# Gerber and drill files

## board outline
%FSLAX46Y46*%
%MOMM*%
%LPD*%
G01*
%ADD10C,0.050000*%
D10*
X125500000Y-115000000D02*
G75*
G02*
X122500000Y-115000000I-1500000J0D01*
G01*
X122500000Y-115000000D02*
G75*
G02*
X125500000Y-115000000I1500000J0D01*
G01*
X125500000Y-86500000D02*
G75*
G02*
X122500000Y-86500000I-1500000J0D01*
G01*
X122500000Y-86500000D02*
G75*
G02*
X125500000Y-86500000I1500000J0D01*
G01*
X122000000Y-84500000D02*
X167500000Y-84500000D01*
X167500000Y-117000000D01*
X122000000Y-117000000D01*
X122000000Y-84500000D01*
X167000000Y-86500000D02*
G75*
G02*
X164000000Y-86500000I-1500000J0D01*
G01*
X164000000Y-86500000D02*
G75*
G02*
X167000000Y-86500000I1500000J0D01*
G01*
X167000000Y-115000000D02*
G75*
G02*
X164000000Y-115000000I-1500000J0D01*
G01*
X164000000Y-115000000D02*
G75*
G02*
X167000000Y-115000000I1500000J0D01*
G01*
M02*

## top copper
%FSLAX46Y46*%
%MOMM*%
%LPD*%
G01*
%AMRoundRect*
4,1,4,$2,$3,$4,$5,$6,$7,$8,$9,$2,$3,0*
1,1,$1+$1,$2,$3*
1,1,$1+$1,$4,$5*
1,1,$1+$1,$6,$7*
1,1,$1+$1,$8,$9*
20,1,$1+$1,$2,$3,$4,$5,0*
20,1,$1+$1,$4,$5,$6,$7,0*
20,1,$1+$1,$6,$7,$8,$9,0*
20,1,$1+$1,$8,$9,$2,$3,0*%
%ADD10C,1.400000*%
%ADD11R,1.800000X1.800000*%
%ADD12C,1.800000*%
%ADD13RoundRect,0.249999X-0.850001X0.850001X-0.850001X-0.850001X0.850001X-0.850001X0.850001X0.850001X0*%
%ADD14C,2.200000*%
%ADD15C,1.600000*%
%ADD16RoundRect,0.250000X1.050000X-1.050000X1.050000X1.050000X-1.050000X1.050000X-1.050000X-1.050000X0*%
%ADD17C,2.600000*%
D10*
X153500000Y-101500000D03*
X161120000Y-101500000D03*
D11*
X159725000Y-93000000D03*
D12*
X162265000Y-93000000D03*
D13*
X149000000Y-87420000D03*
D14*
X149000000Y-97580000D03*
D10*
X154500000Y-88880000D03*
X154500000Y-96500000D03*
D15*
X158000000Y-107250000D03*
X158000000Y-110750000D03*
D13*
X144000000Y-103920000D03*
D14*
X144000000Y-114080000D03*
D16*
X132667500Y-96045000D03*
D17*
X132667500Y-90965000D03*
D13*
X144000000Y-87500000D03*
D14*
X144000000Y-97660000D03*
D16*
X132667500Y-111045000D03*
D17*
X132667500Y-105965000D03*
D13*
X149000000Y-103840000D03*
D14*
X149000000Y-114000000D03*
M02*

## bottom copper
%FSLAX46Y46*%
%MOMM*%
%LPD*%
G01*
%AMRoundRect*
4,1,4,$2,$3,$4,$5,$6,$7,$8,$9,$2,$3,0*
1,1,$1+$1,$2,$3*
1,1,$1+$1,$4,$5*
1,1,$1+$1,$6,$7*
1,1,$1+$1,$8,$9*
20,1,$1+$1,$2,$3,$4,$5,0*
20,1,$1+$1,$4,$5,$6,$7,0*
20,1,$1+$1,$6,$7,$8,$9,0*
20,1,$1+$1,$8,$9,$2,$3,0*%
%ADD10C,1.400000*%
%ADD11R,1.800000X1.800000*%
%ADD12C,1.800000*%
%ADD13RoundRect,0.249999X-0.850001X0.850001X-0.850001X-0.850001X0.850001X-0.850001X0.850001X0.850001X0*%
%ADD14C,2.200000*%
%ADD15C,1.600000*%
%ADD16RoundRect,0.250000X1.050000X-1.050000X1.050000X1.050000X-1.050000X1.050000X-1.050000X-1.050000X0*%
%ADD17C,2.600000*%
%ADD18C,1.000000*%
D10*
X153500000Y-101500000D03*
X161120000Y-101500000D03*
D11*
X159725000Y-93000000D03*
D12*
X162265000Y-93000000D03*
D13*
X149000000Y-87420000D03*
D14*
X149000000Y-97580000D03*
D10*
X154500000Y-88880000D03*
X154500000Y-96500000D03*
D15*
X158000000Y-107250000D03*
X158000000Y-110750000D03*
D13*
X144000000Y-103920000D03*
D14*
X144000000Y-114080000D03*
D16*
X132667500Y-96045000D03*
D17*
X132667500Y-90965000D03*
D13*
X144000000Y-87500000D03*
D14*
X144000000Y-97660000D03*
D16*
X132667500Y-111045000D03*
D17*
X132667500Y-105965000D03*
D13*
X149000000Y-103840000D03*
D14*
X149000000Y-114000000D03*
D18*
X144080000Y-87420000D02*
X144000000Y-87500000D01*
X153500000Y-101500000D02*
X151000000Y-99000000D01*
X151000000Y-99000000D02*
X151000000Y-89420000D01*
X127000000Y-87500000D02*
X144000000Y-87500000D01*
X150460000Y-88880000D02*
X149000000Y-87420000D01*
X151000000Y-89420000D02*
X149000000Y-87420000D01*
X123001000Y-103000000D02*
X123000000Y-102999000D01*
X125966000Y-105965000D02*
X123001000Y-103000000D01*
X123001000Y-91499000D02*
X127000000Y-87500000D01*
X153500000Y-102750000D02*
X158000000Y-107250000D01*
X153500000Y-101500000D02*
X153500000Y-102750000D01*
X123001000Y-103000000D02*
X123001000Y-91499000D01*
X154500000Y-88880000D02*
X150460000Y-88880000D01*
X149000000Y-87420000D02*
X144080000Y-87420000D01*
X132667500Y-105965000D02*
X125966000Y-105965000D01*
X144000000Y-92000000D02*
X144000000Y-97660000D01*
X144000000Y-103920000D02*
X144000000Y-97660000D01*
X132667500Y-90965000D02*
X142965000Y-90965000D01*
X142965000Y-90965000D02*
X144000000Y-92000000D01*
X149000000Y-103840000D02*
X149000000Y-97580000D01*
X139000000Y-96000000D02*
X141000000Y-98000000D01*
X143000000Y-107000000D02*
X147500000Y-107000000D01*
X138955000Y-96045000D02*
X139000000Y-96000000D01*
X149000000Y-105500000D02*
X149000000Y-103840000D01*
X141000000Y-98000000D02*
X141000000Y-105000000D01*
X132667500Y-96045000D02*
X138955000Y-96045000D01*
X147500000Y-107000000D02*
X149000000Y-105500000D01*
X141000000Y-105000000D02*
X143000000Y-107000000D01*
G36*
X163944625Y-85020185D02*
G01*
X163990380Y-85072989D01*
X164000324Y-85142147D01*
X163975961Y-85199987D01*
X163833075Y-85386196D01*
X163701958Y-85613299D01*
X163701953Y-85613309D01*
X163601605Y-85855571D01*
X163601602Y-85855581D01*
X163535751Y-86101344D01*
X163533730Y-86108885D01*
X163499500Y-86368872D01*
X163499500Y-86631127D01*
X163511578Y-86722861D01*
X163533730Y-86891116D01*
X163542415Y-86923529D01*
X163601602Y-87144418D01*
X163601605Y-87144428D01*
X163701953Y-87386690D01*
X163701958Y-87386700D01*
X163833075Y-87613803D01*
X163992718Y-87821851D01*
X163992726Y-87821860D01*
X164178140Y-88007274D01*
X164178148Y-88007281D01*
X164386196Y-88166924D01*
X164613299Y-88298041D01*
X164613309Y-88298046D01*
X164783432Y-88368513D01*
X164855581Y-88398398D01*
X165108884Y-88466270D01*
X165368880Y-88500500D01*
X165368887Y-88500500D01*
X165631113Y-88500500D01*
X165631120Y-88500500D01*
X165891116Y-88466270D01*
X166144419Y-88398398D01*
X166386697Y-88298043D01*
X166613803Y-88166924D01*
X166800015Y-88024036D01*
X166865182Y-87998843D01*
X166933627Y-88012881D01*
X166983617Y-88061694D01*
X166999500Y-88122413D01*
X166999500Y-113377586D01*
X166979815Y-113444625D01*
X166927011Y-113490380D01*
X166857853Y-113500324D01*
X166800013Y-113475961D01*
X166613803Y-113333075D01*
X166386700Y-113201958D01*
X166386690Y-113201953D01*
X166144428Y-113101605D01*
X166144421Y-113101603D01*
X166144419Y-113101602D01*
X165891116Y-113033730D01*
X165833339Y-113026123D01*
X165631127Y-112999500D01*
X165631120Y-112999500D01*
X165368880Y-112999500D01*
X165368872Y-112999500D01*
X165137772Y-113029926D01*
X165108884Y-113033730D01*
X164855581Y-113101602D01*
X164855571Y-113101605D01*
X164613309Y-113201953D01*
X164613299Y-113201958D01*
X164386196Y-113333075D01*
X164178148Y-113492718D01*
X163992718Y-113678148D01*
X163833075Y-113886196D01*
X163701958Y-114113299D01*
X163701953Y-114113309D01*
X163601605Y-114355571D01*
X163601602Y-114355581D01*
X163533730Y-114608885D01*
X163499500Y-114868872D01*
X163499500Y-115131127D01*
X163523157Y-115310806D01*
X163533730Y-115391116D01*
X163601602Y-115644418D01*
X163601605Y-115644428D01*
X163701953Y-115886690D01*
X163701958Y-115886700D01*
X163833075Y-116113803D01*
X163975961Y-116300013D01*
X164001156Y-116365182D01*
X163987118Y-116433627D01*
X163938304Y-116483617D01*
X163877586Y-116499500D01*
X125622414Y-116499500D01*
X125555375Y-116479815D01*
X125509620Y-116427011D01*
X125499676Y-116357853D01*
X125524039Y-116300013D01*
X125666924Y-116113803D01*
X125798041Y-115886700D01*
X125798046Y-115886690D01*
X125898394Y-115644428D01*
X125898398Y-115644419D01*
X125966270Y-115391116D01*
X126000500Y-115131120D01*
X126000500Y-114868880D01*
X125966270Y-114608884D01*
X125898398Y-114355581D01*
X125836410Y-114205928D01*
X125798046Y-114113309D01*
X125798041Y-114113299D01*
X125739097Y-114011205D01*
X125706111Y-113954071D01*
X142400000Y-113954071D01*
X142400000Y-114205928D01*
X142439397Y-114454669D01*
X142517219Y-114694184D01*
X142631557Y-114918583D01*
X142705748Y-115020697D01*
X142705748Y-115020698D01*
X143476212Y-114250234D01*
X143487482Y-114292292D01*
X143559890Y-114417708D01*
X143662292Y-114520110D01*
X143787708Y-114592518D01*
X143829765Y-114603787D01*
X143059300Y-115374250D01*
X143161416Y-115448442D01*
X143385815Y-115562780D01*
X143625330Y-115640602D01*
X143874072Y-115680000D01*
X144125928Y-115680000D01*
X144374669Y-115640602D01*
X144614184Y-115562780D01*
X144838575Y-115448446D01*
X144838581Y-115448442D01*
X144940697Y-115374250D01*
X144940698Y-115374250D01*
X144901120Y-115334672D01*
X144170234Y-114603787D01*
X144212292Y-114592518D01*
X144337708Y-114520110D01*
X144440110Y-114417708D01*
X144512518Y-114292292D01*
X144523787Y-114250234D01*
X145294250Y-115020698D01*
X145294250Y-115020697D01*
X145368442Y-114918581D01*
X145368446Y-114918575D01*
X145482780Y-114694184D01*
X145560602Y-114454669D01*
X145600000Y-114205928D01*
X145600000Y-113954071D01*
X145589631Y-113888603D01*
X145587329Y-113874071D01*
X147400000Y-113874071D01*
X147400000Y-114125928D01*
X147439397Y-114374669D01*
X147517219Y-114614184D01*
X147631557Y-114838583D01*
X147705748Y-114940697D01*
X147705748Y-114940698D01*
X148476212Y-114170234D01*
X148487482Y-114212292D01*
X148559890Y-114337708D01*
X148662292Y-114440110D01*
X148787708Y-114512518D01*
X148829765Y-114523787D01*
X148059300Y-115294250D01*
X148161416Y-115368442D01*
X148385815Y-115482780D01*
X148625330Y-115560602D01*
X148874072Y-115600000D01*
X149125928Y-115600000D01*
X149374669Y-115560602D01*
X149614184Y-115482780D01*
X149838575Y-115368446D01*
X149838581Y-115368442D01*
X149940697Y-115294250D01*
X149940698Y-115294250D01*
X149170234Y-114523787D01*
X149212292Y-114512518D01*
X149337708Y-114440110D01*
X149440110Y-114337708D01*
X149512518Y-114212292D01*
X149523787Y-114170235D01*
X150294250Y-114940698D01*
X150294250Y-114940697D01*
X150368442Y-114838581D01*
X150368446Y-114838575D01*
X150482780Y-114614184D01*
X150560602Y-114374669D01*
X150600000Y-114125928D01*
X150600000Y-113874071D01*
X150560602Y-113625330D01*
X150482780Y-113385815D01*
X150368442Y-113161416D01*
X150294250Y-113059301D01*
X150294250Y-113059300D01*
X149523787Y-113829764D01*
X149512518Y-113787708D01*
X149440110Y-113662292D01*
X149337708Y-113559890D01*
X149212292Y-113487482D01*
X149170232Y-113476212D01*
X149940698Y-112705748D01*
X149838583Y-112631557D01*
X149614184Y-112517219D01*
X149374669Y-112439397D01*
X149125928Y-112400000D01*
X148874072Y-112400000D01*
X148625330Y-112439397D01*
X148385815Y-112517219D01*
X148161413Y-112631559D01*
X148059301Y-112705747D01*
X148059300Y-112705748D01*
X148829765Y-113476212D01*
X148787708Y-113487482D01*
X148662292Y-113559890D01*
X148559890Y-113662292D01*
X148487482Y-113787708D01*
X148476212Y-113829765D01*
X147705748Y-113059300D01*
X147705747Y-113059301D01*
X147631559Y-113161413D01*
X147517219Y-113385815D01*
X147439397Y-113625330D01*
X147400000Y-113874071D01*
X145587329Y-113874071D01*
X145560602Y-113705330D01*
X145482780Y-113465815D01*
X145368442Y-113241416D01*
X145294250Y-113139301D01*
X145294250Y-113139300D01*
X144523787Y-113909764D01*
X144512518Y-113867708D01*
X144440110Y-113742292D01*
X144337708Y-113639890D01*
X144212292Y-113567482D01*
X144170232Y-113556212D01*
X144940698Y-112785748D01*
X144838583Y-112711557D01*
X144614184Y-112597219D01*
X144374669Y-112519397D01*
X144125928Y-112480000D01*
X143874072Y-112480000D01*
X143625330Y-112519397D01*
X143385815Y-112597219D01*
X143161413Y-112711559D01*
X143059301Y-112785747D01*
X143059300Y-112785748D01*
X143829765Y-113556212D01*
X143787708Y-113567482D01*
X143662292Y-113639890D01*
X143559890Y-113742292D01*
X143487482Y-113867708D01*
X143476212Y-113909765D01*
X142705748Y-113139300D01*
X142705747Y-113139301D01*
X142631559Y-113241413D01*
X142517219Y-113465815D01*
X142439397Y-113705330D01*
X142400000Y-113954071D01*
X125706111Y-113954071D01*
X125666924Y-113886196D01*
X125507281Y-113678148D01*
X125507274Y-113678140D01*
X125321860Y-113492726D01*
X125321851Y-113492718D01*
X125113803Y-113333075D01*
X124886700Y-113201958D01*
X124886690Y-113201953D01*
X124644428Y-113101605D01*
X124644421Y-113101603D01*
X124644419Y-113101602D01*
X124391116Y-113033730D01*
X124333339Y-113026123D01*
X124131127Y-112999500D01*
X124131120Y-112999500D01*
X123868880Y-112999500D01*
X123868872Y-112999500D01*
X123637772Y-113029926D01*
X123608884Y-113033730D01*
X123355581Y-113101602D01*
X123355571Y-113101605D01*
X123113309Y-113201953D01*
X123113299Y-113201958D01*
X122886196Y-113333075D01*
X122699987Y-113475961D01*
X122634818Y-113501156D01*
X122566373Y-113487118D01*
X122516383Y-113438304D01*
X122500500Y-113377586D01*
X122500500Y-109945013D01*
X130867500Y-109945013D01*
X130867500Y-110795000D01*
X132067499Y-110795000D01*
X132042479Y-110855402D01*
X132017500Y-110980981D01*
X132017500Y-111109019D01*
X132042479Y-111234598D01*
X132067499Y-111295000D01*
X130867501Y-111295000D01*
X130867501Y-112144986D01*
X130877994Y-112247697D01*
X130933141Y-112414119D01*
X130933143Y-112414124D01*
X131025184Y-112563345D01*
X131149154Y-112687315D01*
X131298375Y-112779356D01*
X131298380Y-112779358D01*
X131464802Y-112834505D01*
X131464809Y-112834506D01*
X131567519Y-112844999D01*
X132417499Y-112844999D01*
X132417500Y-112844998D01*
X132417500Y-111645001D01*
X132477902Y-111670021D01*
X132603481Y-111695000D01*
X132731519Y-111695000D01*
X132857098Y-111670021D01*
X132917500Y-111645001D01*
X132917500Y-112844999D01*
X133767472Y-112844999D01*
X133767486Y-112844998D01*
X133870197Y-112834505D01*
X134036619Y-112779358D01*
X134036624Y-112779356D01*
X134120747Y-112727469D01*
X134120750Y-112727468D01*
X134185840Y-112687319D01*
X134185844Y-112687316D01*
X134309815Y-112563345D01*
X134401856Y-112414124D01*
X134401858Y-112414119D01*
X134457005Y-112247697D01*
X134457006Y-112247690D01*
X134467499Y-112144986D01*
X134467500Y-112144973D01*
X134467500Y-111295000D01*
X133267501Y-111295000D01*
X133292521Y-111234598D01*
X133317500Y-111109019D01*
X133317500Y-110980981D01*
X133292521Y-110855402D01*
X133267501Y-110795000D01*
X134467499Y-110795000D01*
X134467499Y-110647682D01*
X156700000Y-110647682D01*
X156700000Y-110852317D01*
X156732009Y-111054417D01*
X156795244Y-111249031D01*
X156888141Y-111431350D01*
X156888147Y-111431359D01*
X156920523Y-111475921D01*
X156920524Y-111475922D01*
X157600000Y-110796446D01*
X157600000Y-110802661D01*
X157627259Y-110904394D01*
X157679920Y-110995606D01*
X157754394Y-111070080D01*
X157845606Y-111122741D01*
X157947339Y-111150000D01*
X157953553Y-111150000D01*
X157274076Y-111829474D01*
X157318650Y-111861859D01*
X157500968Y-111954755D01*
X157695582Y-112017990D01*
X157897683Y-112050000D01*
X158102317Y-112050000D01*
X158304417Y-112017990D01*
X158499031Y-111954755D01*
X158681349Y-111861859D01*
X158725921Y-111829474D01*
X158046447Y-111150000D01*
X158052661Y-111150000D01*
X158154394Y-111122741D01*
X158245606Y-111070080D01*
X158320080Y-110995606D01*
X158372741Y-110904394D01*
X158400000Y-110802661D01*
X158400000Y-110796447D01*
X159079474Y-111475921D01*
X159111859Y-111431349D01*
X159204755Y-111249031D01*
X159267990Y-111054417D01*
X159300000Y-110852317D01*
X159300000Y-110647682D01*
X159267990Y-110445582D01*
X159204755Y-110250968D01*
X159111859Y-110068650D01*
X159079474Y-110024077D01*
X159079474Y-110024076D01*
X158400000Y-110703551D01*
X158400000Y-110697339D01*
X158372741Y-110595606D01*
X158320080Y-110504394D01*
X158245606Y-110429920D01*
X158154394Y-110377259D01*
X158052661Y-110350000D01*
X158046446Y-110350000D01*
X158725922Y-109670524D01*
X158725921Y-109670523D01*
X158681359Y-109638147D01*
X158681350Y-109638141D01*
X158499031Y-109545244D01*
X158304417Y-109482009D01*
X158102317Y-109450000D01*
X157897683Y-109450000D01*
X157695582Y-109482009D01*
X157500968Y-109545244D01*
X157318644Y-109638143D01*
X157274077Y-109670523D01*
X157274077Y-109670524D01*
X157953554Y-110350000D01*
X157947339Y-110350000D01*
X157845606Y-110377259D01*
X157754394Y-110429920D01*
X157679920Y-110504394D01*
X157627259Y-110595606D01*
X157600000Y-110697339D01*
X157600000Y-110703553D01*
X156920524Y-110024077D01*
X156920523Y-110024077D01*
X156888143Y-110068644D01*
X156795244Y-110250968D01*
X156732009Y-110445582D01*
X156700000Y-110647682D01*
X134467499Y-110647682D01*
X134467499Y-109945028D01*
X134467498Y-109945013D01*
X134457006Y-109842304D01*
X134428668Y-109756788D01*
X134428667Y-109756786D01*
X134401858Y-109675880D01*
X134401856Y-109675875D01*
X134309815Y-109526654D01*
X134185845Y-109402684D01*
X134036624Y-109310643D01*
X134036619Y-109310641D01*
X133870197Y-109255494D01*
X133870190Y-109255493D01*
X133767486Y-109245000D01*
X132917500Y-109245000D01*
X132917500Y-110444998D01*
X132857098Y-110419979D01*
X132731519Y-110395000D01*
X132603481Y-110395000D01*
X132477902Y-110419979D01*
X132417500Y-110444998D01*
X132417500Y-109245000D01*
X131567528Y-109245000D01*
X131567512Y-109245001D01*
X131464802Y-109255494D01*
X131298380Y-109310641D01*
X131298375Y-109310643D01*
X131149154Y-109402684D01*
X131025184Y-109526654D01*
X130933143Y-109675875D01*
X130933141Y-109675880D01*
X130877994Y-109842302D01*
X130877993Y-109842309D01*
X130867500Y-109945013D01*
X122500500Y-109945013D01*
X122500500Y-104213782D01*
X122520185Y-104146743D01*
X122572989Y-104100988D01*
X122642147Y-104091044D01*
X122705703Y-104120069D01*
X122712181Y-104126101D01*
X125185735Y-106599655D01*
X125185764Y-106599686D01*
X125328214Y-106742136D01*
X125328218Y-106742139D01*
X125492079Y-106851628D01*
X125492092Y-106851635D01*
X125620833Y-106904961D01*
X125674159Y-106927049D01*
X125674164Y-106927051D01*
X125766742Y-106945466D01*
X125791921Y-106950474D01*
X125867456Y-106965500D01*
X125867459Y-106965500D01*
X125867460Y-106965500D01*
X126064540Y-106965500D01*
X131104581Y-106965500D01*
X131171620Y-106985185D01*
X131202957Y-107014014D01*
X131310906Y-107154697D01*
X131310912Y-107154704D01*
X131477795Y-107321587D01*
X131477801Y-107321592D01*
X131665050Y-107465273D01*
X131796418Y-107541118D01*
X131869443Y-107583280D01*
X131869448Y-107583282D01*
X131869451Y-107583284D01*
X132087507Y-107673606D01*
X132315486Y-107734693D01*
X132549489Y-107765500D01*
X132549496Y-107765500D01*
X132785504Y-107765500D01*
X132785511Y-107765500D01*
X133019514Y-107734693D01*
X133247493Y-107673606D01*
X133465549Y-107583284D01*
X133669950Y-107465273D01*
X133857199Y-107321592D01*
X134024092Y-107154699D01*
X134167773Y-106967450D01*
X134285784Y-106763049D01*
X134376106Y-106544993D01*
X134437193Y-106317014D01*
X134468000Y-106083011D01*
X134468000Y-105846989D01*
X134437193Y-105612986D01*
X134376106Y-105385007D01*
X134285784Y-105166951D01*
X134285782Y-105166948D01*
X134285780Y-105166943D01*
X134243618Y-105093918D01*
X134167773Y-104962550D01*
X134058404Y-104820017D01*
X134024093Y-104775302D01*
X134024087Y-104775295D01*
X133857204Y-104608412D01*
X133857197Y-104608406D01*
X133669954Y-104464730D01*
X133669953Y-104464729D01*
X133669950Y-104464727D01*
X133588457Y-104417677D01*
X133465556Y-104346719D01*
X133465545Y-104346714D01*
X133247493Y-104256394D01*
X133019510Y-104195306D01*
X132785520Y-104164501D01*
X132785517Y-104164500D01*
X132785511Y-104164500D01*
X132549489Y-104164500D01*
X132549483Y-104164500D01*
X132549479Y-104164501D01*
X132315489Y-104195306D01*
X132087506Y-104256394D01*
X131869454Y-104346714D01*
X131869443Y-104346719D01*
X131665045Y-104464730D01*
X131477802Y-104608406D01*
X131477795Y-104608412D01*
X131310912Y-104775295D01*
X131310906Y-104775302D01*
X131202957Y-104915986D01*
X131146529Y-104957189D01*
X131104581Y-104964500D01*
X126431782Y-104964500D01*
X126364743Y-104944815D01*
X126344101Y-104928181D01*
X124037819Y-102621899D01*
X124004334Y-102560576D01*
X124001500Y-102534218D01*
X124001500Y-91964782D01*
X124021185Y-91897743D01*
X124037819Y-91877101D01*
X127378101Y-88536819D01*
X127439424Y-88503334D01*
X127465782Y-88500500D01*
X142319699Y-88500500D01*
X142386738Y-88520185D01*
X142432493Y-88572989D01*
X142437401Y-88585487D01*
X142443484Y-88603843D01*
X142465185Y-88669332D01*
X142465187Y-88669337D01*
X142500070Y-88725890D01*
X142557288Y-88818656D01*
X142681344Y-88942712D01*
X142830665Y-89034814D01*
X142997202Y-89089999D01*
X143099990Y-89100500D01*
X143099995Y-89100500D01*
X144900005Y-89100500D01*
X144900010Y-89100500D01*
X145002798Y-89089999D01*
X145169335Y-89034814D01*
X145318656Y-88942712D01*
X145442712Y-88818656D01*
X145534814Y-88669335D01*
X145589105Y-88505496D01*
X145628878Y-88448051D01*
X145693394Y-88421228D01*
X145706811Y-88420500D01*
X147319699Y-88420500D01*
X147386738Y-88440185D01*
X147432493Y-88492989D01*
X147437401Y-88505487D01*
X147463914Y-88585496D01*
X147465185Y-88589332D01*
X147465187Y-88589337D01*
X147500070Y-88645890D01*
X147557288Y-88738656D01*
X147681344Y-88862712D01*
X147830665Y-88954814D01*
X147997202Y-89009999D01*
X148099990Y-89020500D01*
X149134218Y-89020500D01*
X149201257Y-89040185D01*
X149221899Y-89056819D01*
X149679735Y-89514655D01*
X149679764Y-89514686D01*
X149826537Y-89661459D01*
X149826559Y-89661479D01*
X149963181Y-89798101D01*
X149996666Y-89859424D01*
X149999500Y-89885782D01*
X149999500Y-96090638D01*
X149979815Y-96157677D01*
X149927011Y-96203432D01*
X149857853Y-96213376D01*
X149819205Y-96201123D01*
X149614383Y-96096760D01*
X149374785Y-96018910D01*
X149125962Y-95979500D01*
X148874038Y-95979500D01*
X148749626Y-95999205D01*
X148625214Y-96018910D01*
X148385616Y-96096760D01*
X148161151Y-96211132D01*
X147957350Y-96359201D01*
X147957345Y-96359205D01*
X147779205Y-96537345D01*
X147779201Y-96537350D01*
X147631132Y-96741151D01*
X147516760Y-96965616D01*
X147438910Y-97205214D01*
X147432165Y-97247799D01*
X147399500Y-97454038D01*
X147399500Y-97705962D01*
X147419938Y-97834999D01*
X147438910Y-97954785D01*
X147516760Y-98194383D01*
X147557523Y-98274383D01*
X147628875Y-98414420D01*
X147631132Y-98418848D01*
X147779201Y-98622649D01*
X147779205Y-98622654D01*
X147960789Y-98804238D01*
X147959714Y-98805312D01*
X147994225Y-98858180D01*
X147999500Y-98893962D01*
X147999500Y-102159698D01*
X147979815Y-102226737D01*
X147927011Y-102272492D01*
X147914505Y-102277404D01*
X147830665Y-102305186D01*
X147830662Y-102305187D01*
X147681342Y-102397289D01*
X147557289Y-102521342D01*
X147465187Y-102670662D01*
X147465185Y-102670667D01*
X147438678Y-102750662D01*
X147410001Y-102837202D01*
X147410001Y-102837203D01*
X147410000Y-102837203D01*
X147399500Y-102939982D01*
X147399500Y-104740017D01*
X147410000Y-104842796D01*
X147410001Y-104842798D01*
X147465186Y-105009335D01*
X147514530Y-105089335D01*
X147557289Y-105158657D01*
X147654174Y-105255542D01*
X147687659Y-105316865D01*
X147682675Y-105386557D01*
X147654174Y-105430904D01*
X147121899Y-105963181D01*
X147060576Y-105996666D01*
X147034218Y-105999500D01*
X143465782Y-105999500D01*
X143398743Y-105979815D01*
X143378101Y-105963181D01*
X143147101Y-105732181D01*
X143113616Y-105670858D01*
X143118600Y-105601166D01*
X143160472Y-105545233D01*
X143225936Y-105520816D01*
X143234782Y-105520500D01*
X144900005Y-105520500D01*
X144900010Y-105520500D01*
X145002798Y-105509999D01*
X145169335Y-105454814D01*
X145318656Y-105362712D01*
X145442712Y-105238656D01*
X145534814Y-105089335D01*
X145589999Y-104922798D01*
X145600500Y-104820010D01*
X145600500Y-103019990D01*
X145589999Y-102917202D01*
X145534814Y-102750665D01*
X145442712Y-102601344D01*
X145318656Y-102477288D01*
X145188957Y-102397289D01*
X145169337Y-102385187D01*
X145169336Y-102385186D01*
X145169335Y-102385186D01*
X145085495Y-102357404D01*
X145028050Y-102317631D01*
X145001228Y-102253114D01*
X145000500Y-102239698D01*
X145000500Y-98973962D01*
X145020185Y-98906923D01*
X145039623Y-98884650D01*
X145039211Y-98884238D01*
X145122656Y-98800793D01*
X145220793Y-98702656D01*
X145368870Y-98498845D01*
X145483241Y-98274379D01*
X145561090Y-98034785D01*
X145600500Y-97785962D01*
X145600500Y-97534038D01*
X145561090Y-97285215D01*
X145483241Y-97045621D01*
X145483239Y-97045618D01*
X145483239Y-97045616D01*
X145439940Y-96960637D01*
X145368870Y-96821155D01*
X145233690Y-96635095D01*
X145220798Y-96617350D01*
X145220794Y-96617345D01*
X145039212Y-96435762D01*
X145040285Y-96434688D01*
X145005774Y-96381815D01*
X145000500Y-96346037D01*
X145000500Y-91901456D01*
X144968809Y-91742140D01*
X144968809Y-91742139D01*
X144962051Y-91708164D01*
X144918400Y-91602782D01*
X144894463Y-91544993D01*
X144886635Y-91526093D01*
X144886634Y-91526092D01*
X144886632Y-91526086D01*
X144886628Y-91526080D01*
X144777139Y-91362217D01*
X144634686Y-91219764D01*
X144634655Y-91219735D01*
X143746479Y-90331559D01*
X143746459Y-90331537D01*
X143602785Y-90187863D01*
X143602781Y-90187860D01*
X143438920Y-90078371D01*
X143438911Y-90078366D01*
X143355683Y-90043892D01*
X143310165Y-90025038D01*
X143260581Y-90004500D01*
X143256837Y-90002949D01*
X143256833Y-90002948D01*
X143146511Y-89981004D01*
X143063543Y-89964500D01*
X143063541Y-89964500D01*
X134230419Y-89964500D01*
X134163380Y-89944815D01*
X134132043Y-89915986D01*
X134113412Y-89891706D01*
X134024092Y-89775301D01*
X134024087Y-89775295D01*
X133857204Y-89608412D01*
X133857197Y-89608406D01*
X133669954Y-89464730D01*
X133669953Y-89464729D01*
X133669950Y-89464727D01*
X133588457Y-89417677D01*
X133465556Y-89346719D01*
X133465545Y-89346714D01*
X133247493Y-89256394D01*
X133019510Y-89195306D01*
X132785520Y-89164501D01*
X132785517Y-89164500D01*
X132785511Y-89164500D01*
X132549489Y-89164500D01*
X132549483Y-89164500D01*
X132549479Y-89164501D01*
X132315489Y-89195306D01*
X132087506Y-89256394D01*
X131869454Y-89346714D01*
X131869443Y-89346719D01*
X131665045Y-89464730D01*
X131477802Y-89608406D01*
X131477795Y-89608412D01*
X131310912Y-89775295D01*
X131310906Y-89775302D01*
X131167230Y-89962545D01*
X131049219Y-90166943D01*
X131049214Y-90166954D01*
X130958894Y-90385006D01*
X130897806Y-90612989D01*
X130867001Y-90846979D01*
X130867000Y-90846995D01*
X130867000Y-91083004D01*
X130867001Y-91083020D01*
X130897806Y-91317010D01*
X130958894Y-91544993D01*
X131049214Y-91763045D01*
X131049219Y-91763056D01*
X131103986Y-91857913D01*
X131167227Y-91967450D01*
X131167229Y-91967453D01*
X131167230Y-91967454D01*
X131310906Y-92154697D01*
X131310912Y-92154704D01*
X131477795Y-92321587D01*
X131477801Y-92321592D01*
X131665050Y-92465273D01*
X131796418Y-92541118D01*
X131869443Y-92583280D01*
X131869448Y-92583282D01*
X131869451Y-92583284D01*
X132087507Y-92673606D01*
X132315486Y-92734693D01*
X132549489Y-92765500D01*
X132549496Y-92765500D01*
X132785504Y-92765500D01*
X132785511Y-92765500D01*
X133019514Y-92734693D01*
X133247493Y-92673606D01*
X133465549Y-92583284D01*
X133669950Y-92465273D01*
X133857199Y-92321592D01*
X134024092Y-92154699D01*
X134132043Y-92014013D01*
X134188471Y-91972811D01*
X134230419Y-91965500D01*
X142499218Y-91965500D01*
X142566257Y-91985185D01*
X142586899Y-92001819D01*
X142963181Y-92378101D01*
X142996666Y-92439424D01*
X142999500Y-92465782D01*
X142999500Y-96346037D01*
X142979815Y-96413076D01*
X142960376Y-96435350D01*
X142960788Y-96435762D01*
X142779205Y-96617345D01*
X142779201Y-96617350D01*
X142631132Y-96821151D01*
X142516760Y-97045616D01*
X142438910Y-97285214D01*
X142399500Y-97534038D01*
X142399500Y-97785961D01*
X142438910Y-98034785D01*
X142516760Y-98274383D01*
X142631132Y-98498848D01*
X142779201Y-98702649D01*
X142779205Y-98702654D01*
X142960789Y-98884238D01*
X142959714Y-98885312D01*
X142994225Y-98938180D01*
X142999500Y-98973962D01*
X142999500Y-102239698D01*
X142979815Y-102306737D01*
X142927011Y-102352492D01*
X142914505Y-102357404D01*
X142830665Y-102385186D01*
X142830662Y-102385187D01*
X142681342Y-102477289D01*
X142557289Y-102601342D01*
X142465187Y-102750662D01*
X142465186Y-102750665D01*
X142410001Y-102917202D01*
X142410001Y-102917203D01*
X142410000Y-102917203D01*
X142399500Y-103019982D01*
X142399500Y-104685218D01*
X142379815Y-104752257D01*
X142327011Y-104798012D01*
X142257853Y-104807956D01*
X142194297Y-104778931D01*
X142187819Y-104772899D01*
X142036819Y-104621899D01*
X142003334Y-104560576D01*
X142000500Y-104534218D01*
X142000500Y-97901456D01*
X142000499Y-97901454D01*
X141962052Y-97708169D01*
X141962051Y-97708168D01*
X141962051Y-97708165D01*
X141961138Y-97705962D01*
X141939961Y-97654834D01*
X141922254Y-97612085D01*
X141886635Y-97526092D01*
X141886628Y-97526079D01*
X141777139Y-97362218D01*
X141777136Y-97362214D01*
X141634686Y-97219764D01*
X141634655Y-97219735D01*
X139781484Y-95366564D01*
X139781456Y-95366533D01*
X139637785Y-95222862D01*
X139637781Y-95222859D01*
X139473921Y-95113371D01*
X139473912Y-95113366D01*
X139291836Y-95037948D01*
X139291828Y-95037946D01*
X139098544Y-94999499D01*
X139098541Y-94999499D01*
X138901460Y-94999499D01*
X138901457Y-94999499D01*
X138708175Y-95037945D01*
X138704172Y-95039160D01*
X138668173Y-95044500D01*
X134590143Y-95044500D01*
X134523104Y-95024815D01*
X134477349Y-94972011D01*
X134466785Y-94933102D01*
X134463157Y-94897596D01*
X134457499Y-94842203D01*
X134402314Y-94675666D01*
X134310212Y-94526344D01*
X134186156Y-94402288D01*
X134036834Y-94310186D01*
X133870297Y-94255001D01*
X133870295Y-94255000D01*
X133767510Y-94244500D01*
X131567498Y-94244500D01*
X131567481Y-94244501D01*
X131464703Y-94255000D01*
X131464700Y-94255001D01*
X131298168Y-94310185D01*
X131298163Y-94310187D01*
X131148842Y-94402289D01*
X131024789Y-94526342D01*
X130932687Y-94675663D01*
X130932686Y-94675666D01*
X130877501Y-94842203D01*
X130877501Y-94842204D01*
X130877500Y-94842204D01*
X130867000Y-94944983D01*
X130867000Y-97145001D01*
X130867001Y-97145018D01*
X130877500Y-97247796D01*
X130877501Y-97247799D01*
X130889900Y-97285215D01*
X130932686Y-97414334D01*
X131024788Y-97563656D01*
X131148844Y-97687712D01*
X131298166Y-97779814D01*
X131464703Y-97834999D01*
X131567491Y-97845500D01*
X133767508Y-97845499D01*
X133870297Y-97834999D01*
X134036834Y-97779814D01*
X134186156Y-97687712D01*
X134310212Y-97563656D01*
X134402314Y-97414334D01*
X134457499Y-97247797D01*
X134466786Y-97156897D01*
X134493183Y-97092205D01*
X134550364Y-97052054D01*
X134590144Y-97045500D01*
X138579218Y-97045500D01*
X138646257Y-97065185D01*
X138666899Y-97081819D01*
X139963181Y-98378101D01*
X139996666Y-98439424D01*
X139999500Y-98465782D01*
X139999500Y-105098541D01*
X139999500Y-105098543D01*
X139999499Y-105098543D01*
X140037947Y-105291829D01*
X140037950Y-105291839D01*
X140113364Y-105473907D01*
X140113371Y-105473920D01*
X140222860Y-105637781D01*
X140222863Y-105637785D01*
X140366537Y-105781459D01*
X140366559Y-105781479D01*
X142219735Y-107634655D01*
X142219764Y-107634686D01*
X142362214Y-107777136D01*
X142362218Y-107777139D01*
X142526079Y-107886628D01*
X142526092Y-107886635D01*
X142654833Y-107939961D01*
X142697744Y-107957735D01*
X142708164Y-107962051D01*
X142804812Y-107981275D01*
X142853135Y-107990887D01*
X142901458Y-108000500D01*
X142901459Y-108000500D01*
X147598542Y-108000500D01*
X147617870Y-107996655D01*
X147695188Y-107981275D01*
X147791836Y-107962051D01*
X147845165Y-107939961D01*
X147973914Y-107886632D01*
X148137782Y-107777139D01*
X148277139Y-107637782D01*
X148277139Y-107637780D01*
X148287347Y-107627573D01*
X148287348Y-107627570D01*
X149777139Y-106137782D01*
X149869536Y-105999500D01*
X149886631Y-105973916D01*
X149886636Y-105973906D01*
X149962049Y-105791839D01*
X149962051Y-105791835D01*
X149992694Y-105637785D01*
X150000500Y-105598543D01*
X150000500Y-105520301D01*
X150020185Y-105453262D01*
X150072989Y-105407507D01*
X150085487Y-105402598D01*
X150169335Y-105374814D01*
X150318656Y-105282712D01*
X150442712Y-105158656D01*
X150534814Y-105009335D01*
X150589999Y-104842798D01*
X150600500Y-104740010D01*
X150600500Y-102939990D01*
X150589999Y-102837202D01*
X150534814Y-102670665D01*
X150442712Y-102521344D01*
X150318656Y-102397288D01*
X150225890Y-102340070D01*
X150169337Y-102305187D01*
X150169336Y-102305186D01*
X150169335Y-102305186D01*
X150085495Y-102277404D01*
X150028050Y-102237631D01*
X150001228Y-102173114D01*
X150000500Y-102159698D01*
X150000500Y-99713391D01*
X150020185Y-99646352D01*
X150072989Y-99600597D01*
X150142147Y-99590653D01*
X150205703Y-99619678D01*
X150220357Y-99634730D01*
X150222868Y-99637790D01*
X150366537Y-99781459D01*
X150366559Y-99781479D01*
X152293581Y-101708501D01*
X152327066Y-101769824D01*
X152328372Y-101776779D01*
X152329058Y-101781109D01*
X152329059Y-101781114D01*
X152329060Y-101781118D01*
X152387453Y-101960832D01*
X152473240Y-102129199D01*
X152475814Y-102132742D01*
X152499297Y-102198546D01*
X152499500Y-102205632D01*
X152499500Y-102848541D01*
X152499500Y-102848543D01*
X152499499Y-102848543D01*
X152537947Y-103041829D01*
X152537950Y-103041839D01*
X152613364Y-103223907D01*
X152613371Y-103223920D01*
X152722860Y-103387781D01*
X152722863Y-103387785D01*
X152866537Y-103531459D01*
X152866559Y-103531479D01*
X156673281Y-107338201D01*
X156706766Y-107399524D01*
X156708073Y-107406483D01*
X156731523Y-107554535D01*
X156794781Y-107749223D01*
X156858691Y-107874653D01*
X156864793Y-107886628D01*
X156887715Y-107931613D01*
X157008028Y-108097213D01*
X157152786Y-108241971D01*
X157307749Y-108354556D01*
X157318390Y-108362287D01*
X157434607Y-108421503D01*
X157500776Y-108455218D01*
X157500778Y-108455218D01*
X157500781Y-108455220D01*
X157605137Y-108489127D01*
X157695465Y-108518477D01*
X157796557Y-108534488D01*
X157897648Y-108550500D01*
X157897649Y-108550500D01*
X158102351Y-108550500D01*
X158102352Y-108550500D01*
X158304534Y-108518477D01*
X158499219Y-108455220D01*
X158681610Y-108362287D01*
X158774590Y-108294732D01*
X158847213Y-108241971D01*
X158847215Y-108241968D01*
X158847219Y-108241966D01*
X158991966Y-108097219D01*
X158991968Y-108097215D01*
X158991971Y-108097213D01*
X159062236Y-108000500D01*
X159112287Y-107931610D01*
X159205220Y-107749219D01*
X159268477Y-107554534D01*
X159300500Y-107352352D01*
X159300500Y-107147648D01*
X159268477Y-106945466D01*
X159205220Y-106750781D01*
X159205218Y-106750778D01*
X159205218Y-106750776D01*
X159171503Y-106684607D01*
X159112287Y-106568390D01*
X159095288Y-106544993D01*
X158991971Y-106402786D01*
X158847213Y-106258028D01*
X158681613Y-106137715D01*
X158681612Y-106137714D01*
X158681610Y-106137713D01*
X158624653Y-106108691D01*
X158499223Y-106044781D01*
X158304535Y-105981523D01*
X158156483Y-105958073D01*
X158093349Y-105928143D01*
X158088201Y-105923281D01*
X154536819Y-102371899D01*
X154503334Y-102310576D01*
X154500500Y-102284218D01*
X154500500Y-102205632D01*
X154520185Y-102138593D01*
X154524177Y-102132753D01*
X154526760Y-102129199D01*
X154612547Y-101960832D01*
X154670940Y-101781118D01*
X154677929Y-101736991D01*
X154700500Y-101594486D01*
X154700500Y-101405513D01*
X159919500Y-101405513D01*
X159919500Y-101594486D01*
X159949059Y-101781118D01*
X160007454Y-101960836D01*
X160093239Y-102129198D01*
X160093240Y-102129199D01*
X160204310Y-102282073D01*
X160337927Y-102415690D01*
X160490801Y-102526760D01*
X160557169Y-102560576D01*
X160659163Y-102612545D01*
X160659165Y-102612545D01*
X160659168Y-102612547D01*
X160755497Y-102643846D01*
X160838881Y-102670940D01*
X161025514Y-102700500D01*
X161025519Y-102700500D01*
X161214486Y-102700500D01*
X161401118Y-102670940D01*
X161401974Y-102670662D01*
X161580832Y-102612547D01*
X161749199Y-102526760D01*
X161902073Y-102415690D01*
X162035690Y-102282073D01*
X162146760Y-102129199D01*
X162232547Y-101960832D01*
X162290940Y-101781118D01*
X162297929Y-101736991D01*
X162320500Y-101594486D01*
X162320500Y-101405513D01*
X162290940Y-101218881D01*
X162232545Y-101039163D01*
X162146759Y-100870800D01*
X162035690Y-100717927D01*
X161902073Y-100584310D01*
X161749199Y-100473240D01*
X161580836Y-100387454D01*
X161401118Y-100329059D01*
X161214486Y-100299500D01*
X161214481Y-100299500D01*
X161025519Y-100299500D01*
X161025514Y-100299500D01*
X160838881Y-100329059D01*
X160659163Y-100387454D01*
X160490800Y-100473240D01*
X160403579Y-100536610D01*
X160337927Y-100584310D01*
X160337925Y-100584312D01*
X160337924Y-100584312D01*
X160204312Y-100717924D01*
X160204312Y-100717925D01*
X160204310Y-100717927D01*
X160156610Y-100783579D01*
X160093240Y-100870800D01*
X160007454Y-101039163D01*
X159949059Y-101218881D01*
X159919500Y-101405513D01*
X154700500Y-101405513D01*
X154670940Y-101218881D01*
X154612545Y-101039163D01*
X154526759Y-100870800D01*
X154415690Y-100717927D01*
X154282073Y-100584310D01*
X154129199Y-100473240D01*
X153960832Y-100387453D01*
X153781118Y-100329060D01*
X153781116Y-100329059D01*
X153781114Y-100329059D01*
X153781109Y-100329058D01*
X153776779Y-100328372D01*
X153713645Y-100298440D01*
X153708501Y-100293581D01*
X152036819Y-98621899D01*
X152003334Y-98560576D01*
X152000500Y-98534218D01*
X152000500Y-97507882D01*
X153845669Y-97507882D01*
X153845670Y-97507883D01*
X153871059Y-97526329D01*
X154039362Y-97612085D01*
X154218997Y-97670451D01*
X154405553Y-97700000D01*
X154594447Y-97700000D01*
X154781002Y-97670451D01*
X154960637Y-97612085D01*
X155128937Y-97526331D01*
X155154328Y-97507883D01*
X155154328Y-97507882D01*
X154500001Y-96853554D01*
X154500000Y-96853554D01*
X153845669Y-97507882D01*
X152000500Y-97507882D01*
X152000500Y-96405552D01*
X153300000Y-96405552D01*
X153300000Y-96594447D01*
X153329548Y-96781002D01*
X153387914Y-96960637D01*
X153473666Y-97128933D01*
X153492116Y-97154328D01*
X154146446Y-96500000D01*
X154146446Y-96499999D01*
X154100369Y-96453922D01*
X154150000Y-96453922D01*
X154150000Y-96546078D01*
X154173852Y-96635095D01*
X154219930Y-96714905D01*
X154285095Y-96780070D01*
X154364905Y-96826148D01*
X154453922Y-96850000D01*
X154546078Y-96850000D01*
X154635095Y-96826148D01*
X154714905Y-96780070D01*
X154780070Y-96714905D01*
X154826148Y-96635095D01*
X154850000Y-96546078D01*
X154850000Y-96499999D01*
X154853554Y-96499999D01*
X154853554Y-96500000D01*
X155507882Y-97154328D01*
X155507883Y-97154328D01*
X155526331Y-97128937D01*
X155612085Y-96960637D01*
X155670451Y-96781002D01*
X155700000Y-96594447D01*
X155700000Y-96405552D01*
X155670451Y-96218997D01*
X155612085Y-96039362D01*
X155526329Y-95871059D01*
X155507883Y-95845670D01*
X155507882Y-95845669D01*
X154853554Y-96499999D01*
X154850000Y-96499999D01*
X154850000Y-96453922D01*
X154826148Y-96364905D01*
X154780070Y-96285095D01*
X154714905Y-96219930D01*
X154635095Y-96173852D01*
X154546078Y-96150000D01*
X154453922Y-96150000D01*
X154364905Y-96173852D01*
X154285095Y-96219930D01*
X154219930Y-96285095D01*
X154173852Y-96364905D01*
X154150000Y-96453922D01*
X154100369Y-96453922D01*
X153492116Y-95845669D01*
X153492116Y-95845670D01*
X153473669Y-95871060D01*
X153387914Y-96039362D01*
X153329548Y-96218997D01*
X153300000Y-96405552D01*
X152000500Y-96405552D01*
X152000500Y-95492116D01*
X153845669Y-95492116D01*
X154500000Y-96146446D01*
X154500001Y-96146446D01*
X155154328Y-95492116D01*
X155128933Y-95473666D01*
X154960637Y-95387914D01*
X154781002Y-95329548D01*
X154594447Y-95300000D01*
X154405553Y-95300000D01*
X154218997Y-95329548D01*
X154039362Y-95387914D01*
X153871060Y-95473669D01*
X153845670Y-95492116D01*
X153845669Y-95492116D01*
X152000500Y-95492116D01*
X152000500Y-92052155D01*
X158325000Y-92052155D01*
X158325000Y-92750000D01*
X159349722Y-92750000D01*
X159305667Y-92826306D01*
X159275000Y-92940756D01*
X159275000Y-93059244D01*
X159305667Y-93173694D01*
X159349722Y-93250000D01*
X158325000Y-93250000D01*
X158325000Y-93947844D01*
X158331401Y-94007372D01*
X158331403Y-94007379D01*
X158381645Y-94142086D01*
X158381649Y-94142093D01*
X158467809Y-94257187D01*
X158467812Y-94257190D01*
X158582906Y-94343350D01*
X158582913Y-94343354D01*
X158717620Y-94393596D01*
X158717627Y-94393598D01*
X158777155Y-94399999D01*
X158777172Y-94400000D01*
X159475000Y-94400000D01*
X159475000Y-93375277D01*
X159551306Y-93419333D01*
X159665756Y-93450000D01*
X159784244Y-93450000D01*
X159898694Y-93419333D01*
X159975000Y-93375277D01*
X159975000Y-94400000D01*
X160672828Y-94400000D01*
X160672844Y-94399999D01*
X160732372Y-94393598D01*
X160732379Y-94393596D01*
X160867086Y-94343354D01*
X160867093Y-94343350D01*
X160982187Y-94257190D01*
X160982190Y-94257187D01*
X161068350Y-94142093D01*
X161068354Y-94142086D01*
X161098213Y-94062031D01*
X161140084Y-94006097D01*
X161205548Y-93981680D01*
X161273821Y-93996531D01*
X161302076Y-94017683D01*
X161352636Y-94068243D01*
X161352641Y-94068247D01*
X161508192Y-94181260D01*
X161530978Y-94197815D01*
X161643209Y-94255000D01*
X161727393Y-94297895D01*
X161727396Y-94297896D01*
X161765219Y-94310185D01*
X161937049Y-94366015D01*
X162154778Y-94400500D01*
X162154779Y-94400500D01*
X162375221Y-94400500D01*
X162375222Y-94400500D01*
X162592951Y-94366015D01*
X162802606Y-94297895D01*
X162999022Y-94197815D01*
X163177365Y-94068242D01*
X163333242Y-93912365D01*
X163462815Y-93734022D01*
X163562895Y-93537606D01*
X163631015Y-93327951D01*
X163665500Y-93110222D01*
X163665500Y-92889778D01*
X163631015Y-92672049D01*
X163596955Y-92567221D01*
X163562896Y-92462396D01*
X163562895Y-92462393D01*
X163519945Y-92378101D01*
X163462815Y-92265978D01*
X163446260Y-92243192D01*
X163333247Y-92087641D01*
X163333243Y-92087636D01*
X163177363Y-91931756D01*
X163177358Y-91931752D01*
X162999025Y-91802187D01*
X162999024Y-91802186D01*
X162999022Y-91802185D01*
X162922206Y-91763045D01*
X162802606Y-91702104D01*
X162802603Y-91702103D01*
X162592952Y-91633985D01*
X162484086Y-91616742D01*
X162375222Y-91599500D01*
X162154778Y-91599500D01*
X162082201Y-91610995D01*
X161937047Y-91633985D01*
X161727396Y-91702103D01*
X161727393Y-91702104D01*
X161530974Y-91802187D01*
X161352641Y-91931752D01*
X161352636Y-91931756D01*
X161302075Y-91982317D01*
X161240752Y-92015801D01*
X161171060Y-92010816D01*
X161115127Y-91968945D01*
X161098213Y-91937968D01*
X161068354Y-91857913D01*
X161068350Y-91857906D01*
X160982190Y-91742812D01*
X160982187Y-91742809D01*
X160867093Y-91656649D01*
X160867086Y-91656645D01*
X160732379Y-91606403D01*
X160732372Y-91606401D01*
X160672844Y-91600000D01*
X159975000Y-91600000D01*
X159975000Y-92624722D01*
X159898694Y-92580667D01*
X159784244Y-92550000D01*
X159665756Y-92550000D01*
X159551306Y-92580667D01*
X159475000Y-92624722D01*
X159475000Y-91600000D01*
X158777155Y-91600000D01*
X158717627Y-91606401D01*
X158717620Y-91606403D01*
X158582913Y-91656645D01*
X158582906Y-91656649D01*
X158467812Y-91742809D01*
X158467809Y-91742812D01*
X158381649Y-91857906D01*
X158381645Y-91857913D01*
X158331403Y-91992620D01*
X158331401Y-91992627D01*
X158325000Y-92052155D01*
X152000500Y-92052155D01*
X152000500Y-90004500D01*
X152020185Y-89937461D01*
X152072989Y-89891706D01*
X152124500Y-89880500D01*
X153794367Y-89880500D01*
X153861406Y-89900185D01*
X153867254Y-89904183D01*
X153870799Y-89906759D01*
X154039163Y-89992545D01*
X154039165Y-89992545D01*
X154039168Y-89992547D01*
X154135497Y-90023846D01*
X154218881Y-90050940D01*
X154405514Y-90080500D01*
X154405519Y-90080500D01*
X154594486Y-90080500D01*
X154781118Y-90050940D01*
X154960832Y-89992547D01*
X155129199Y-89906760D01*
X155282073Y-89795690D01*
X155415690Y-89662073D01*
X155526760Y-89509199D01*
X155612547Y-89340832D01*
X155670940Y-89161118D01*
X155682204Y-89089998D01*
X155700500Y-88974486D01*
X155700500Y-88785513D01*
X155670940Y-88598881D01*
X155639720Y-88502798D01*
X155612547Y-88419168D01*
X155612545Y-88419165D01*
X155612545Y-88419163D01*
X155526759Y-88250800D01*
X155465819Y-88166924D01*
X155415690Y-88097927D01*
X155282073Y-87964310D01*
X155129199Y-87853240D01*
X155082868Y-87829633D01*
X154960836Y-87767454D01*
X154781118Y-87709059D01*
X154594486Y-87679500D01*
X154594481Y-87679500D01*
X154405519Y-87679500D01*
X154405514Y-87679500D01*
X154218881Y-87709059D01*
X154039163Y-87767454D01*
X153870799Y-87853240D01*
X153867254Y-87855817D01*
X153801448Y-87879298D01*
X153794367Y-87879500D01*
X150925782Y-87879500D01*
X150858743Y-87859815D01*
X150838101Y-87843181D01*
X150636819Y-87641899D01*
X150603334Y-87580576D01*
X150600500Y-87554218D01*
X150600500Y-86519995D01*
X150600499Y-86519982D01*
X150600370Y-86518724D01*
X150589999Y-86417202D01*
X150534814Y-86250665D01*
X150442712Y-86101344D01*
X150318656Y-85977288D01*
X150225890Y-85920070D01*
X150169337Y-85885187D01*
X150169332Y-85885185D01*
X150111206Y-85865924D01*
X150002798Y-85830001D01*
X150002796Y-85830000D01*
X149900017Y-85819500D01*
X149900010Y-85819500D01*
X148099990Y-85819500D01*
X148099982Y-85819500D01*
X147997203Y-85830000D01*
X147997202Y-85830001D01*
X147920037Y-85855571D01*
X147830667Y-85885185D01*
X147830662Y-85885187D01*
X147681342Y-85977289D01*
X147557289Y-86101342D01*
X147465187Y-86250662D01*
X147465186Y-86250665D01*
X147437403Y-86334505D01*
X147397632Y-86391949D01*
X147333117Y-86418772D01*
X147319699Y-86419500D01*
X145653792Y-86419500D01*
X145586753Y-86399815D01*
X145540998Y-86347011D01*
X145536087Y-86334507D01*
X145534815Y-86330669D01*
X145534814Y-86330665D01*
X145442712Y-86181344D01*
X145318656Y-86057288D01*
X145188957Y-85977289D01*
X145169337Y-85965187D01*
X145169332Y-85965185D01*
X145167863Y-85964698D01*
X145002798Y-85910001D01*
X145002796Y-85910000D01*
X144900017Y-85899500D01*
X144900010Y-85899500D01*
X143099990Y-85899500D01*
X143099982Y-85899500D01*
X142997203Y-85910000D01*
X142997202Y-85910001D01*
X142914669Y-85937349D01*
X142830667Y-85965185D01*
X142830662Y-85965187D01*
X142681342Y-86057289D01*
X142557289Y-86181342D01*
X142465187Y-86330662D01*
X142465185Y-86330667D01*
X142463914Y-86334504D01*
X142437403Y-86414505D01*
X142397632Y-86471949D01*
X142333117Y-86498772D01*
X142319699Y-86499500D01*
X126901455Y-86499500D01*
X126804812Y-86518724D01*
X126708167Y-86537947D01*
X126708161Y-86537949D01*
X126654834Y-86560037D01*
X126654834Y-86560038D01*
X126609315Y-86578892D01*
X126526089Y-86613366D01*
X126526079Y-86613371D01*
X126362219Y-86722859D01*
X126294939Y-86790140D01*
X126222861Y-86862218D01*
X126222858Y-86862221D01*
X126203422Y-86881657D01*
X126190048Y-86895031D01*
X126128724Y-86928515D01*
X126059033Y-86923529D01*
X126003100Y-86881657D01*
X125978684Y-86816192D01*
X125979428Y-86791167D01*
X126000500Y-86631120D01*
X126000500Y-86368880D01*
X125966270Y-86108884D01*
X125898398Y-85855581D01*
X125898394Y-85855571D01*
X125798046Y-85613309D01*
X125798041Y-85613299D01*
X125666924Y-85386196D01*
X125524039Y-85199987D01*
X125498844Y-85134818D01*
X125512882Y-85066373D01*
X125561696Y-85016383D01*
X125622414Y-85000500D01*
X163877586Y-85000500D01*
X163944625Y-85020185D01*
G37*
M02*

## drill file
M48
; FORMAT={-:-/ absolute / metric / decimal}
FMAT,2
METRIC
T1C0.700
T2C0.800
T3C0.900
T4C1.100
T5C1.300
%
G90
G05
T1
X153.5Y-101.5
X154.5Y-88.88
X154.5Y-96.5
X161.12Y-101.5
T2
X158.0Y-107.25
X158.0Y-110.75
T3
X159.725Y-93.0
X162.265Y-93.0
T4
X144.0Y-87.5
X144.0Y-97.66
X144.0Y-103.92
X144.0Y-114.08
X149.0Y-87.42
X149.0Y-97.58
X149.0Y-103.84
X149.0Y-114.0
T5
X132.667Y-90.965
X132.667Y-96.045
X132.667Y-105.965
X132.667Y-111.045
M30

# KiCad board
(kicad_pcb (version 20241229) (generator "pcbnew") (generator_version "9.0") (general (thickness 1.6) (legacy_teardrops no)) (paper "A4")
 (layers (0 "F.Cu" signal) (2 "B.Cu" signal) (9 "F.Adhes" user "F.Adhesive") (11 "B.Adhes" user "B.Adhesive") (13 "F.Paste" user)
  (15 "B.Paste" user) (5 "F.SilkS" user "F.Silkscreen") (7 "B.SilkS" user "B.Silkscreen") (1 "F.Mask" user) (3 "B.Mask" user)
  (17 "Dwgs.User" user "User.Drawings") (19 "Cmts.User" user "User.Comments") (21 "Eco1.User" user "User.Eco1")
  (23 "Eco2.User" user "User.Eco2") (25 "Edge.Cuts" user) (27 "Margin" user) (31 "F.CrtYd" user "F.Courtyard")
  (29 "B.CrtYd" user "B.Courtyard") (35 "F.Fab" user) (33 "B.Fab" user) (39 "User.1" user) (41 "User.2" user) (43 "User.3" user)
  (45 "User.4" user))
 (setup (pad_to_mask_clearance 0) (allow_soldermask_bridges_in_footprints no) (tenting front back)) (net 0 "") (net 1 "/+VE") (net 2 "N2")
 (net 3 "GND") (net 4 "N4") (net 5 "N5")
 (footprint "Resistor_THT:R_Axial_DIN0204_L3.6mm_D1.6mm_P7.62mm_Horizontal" (layer "F.Cu") (at 153.5 101.5)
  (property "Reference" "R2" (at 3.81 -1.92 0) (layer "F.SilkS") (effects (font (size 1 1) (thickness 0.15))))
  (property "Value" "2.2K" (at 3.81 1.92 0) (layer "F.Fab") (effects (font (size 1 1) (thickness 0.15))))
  (pad "1" thru_hole circle (at 0 0) (size 1.4 1.4) (drill 0.7) (layers "*.Cu" "*.Mask") (remove_unused_layers no) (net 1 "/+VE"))
  (pad "2" thru_hole circle (at 7.62 0) (size 1.4 1.4) (drill 0.7) (layers "*.Cu" "*.Mask") (remove_unused_layers no) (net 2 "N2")))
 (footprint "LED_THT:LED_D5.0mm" (layer "F.Cu") (at 159.725 93)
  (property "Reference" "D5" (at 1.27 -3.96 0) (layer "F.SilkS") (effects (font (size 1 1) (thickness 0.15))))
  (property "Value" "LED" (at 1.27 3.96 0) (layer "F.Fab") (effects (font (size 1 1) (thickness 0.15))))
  (pad "1" thru_hole rect (at 0 0) (size 1.8 1.8) (drill 0.9) (layers "*.Cu" "*.Mask") (remove_unused_layers no) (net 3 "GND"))
  (pad "2" thru_hole circle (at 2.54 0) (size 1.8 1.8) (drill 0.9) (layers "*.Cu" "*.Mask") (remove_unused_layers no) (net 2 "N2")))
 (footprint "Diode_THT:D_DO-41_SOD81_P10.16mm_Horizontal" (layer "F.Cu") (at 149 87.42 -90)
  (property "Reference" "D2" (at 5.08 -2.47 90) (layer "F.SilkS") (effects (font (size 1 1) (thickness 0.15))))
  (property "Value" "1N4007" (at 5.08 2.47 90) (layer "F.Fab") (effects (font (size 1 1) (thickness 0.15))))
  (pad "1" thru_hole roundrect (at 0 0 270) (size 2.2 2.2) (drill 1.1) (layers "*.Cu" "*.Mask") (remove_unused_layers no)
   (roundrect_rratio 0.113636) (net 1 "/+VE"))
  (pad "2" thru_hole circle (at 10.16 0 270) (size 2.2 2.2) (drill 1.1) (layers "*.Cu" "*.Mask") (remove_unused_layers no) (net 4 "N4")))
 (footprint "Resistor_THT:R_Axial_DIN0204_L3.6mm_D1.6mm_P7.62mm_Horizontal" (layer "F.Cu") (at 154.5 88.88 -90)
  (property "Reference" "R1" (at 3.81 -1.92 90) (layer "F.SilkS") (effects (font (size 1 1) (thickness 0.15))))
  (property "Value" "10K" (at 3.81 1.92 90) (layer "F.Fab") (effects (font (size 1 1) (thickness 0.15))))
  (pad "1" thru_hole circle (at 0 0 270) (size 1.4 1.4) (drill 0.7) (layers "*.Cu" "*.Mask") (remove_unused_layers no) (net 1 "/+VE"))
  (pad "2" thru_hole circle (at 7.62 0 270) (size 1.4 1.4) (drill 0.7) (layers "*.Cu" "*.Mask") (remove_unused_layers no) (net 3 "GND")))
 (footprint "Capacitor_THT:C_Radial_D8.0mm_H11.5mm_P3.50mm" (layer "F.Cu") (at 158 107.25 -90)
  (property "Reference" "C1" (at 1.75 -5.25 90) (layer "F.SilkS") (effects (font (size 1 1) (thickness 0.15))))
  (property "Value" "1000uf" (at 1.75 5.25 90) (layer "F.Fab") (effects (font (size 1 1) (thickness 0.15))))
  (pad "1" thru_hole circle (at 0 0 270) (size 1.6 1.6) (drill 0.8) (layers "*.Cu" "*.Mask") (remove_unused_layers no) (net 1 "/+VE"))
  (pad "2" thru_hole circle (at 3.5 0 270) (size 1.6 1.6) (drill 0.8) (layers "*.Cu" "*.Mask") (remove_unused_layers no) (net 3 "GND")))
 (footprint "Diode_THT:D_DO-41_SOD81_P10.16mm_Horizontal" (layer "F.Cu") (at 144 103.92 -90)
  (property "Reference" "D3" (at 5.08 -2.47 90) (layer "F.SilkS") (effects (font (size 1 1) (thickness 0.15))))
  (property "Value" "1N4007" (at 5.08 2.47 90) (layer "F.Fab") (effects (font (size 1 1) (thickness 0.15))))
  (pad "1" thru_hole roundrect (at 0 0 270) (size 2.2 2.2) (drill 1.1) (layers "*.Cu" "*.Mask") (remove_unused_layers no)
   (roundrect_rratio 0.113636) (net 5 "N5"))
  (pad "2" thru_hole circle (at 10.16 0 270) (size 2.2 2.2) (drill 1.1) (layers "*.Cu" "*.Mask") (remove_unused_layers no) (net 3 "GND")))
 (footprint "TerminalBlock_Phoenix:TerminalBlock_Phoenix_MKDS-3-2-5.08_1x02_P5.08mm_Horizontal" (layer "F.Cu") (at 132.6675 96.045 90)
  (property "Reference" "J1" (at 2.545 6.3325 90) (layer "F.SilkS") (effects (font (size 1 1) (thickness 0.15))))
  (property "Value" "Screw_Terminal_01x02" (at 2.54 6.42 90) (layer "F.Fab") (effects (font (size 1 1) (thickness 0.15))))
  (pad "1" thru_hole roundrect (at 0 0 90) (size 2.6 2.6) (drill 1.3) (layers "*.Cu" "*.Mask") (remove_unused_layers no)
   (roundrect_rratio 0.096154) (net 4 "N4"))
  (pad "2" thru_hole circle (at 5.08 0 90) (size 2.6 2.6) (drill 1.3) (layers "*.Cu" "*.Mask") (remove_unused_layers no) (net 5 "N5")))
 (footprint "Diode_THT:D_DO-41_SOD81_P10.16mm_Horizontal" (layer "F.Cu") (at 144 87.5 -90)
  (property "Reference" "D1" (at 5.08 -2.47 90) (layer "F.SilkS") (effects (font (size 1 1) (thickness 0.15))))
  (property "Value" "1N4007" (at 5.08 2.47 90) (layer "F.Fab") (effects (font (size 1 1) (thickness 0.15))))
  (pad "1" thru_hole roundrect (at 0 0 270) (size 2.2 2.2) (drill 1.1) (layers "*.Cu" "*.Mask") (remove_unused_layers no)
   (roundrect_rratio 0.113636) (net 1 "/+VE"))
  (pad "2" thru_hole circle (at 10.16 0 270) (size 2.2 2.2) (drill 1.1) (layers "*.Cu" "*.Mask") (remove_unused_layers no) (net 5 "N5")))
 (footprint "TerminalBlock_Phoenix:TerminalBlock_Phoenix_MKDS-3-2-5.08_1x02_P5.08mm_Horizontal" (layer "F.Cu") (at 132.6675 111.045 90)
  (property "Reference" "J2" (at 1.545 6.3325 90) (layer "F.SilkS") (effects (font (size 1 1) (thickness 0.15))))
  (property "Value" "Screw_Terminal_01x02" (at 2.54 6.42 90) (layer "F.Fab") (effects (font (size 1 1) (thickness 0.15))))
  (pad "1" thru_hole roundrect (at 0 0 90) (size 2.6 2.6) (drill 1.3) (layers "*.Cu" "*.Mask") (remove_unused_layers no)
   (roundrect_rratio 0.096154) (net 3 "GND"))
  (pad "2" thru_hole circle (at 5.08 0 90) (size 2.6 2.6) (drill 1.3) (layers "*.Cu" "*.Mask") (remove_unused_layers no) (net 1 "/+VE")))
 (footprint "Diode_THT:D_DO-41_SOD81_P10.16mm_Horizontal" (layer "F.Cu") (at 149 103.84 -90)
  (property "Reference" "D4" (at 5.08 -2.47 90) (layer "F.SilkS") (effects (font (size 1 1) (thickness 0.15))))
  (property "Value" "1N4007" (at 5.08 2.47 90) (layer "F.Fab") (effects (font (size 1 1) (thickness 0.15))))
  (pad "1" thru_hole roundrect (at 0 0 270) (size 2.2 2.2) (drill 1.1) (layers "*.Cu" "*.Mask") (remove_unused_layers no)
   (roundrect_rratio 0.113636) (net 4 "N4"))
  (pad "2" thru_hole circle (at 10.16 0 270) (size 2.2 2.2) (drill 1.1) (layers "*.Cu" "*.Mask") (remove_unused_layers no) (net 3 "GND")))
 (gr_circle (center 124 115) (end 124 116.5) (stroke (width 0.05) (type default)) (fill no) (layer "Edge.Cuts"))
 (gr_circle (center 124 86.5) (end 124 85) (stroke (width 0.05) (type default)) (fill no) (layer "Edge.Cuts"))
 (gr_rect (start 122 84.5) (end 167.5 117) (stroke (width 0.05) (type default)) (fill no) (layer "Edge.Cuts"))
 (gr_circle (center 165.5 86.5) (end 165.5 85) (stroke (width 0.05) (type default)) (fill no) (layer "Edge.Cuts"))
 (gr_circle (center 165.5 115) (end 165.5 116.5) (stroke (width 0.05) (type default)) (fill no) (layer "Edge.Cuts"))
 (segment (start 144.08 87.42) (end 144 87.5) (width 1) (layer "B.Cu") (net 1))
 (segment (start 153.5 101.5) (end 151 99) (width 1) (layer "B.Cu") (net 1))
 (segment (start 151 99) (end 151 89.42) (width 1) (layer "B.Cu") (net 1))
 (segment (start 127 87.5) (end 144 87.5) (width 1) (layer "B.Cu") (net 1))
 (segment (start 150.46 88.88) (end 149 87.42) (width 1) (layer "B.Cu") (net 1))
 (segment (start 151 89.42) (end 149 87.42) (width 1) (layer "B.Cu") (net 1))
 (segment (start 123.001 103) (end 123 102.999) (width 1) (layer "B.Cu") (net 1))
 (segment (start 125.966 105.965) (end 123.001 103) (width 1) (layer "B.Cu") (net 1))
 (segment (start 123.001 91.499) (end 127 87.5) (width 1) (layer "B.Cu") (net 1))
 (segment (start 153.5 102.75) (end 158 107.25) (width 1) (layer "B.Cu") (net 1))
 (segment (start 153.5 101.5) (end 153.5 102.75) (width 1) (layer "B.Cu") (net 1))
 (segment (start 123.001 103) (end 123.001 91.499) (width 1) (layer "B.Cu") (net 1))
 (segment (start 154.5 88.88) (end 150.46 88.88) (width 1) (layer "B.Cu") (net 1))
 (segment (start 149 87.42) (end 144.08 87.42) (width 1) (layer "B.Cu") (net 1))
 (segment (start 132.6675 105.965) (end 125.966 105.965) (width 1) (layer "B.Cu") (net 1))
 (segment (start 144 92) (end 144 97.66) (width 1) (layer "B.Cu") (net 5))
 (segment (start 144 103.92) (end 144 97.66) (width 1) (layer "B.Cu") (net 5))
 (segment (start 132.6675 90.965) (end 142.965 90.965) (width 1) (layer "B.Cu") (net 5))
 (segment (start 142.965 90.965) (end 144 92) (width 1) (layer "B.Cu") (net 5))
 (segment (start 149 103.84) (end 149 97.58) (width 1) (layer "B.Cu") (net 4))
 (segment (start 139 96) (end 141 98) (width 1) (layer "B.Cu") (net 4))
 (segment (start 143 107) (end 147.5 107) (width 1) (layer "B.Cu") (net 4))
 (segment (start 138.955 96.045) (end 139 96) (width 1) (layer "B.Cu") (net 4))
 (segment (start 149 105.5) (end 149 103.84) (width 1) (layer "B.Cu") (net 4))
 (segment (start 141 98) (end 141 105) (width 1) (layer "B.Cu") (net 4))
 (segment (start 132.6675 96.045) (end 138.955 96.045) (width 1) (layer "B.Cu") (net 4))
 (segment (start 147.5 107) (end 149 105.5) (width 1) (layer "B.Cu") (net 4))
 (segment (start 141 105) (end 143 107) (width 1) (layer "B.Cu") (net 4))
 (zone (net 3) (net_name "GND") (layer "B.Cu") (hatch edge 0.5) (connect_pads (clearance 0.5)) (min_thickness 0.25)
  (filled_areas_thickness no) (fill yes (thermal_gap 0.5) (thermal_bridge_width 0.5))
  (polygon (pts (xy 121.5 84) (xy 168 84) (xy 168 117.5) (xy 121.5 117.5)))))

